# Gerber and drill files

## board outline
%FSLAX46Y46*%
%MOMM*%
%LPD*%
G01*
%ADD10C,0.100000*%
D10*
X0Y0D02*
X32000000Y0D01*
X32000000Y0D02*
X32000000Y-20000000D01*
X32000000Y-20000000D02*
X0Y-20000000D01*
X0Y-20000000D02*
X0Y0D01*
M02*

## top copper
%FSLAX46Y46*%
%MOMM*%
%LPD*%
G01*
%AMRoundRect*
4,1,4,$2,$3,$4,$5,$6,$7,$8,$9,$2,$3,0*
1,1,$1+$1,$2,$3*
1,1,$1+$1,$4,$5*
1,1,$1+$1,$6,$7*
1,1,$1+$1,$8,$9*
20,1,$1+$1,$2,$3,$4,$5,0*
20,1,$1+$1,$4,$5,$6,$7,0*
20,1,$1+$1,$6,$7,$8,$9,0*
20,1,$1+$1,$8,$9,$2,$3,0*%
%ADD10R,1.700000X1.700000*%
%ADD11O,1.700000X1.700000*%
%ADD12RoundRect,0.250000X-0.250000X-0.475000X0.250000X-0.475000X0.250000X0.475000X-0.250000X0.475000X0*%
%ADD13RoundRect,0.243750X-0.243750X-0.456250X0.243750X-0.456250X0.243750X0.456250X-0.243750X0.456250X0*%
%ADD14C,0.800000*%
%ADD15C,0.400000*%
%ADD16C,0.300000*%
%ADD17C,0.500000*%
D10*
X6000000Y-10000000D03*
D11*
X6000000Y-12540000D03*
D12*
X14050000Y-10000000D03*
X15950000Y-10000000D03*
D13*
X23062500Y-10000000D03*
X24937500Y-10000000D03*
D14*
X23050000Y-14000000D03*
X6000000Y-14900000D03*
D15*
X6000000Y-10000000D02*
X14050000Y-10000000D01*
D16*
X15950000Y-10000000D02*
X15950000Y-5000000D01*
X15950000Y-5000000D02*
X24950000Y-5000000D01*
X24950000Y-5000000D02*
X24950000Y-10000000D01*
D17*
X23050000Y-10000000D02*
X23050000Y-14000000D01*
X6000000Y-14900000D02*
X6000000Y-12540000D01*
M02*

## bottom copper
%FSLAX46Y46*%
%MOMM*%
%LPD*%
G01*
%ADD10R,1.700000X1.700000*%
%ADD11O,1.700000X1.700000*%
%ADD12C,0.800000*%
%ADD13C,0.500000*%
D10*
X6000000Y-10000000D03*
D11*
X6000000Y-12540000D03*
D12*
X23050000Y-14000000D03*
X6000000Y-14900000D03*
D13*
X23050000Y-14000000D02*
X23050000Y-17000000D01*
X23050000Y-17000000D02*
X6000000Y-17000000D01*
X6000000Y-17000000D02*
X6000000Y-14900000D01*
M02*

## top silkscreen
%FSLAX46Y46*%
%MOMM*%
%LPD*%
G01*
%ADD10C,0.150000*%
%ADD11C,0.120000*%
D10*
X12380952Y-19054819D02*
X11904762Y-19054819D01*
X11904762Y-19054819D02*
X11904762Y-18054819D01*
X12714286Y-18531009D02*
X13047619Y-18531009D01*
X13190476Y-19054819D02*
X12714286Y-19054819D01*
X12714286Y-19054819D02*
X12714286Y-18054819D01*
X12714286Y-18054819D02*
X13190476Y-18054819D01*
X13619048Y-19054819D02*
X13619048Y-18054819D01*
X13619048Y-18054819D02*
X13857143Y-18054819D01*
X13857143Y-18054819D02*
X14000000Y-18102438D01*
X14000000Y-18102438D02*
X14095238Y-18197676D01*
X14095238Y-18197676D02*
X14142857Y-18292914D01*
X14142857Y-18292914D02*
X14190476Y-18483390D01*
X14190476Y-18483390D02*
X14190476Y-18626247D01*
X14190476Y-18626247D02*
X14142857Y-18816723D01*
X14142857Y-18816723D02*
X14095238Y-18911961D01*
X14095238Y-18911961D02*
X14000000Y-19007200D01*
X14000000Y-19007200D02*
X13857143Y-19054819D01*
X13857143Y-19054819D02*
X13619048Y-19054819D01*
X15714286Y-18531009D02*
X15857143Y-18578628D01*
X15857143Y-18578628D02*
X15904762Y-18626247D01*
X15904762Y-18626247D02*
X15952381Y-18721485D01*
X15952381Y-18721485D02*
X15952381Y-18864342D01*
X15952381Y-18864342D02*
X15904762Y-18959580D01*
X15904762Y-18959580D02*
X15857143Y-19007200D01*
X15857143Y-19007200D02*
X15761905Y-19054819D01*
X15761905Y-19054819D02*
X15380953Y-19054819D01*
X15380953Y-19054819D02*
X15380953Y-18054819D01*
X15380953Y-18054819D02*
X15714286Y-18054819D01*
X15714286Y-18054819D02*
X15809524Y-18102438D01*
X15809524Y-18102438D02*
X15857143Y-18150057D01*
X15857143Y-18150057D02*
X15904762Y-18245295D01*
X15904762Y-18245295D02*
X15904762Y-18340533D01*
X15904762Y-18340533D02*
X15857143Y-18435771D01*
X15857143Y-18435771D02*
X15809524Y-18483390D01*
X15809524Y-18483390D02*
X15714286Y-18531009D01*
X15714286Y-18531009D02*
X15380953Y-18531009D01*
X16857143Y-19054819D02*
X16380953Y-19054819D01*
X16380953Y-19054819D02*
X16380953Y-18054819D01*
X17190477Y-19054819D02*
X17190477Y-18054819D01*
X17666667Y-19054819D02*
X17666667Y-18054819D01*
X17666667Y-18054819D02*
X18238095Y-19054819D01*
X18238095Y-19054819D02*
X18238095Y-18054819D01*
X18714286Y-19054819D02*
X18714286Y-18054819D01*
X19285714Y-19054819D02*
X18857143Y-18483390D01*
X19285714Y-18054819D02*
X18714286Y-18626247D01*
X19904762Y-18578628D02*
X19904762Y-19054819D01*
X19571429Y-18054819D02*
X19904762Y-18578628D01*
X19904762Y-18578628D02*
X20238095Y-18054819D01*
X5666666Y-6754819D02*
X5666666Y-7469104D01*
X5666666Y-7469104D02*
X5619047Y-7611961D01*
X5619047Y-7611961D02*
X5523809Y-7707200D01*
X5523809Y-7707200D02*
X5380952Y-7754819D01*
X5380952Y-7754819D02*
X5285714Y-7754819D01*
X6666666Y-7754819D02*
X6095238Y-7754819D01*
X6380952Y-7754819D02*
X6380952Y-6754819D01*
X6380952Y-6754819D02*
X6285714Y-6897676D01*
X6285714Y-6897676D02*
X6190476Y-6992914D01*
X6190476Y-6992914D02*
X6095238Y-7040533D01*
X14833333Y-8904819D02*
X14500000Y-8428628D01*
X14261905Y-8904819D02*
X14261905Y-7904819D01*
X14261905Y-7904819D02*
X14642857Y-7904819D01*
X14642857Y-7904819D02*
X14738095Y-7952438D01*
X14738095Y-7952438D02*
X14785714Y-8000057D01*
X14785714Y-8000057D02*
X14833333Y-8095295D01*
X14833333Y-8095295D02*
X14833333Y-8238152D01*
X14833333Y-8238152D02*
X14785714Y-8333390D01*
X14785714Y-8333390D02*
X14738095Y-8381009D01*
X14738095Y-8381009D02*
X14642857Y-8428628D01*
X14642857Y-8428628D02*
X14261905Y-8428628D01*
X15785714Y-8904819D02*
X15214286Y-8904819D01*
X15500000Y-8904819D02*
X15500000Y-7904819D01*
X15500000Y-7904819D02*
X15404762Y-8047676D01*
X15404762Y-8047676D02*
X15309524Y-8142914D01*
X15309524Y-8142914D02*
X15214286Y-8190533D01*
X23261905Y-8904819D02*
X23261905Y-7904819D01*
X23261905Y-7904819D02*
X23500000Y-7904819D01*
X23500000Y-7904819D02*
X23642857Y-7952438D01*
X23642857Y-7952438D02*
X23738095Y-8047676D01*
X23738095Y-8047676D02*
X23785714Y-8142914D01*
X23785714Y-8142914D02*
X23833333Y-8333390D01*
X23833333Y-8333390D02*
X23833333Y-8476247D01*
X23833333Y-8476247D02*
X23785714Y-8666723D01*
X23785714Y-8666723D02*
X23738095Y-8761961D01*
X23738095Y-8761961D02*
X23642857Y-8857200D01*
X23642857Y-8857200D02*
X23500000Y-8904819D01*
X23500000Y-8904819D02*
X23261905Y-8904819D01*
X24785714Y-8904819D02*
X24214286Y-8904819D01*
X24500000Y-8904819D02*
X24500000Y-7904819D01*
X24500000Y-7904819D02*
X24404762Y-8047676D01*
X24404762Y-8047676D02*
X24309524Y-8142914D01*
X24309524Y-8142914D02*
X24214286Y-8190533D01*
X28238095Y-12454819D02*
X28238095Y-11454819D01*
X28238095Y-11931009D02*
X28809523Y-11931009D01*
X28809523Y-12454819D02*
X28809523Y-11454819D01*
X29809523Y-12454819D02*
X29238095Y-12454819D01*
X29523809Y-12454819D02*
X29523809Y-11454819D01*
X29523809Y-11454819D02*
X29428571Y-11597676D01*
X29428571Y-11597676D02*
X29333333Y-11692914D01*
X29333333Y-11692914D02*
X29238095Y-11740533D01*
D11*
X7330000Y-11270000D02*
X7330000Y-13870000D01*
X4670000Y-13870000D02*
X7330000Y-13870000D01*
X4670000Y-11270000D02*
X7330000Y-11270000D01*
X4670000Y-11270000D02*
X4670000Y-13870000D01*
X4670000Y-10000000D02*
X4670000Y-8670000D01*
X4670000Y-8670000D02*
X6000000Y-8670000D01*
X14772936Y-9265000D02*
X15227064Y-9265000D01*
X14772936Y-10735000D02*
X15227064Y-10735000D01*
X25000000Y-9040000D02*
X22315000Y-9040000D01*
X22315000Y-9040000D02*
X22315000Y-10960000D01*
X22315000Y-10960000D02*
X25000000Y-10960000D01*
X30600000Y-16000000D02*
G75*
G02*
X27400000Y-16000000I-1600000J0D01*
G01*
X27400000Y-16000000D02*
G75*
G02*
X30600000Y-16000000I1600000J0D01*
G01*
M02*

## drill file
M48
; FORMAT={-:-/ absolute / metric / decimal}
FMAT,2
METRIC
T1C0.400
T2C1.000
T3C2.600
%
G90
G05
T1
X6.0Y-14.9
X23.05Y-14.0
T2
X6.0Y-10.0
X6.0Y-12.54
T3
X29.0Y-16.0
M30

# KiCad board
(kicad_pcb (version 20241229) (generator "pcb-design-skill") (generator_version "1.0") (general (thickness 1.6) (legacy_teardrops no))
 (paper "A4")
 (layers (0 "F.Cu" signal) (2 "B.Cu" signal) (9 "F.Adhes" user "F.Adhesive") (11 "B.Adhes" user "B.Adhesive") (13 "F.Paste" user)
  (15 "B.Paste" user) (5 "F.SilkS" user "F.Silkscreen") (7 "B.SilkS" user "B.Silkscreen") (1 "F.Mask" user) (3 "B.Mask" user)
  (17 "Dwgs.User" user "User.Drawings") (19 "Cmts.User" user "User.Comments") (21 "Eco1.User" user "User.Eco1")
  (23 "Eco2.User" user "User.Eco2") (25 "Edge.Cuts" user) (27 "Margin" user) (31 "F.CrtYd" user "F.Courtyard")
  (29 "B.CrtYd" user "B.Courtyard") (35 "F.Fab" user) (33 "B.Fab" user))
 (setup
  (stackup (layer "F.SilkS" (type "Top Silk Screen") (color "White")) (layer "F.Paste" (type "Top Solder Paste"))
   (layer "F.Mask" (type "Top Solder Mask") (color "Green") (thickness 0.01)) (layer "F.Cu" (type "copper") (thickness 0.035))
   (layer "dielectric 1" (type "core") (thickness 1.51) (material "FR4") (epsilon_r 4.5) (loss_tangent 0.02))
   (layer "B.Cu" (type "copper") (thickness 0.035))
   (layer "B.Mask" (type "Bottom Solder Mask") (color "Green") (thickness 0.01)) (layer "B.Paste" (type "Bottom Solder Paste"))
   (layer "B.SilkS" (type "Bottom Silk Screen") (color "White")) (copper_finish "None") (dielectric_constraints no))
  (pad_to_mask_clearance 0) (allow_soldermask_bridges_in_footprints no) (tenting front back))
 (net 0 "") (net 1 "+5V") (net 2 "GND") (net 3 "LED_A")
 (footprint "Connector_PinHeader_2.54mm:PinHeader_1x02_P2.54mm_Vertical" (layer "F.Cu") (at 6 10 0)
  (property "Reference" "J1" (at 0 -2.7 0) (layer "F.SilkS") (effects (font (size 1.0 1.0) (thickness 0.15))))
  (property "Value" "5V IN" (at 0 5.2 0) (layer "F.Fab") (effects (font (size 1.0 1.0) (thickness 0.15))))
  (fp_line (start 1.33 1.27) (end 1.33 3.87) (stroke (width 0.12) (type solid)) (layer "F.SilkS"))
  (fp_line (start -1.33 3.87) (end 1.33 3.87) (stroke (width 0.12) (type solid)) (layer "F.SilkS"))
  (fp_line (start -1.33 1.27) (end 1.33 1.27) (stroke (width 0.12) (type solid)) (layer "F.SilkS"))
  (fp_line (start -1.33 1.27) (end -1.33 3.87) (stroke (width 0.12) (type solid)) (layer "F.SilkS"))
  (fp_line (start -1.33 0) (end -1.33 -1.33) (stroke (width 0.12) (type solid)) (layer "F.SilkS"))
  (fp_line (start -1.33 -1.33) (end 0 -1.33) (stroke (width 0.12) (type solid)) (layer "F.SilkS"))
  (pad "1" thru_hole rect (at 0 0) (size 1.7 1.7) (drill 1) (layers "*.Cu" "*.Mask") (remove_unused_layers no) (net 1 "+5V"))
  (pad "2" thru_hole oval (at 0 2.54) (size 1.7 1.7) (drill 1) (layers "*.Cu" "*.Mask") (remove_unused_layers no) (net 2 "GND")))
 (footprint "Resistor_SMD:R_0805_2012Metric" (layer "F.Cu") (at 15 10)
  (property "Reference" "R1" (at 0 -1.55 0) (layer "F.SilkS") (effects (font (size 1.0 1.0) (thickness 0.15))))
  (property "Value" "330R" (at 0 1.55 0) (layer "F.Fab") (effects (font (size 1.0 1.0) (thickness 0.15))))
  (fp_line (start -0.227064 -0.735) (end 0.227064 -0.735) (stroke (width 0.12) (type solid)) (layer "F.SilkS"))
  (fp_line (start -0.227064 0.735) (end 0.227064 0.735) (stroke (width 0.12) (type solid)) (layer "F.SilkS"))
  (pad "1" smd roundrect (at -0.95 0) (size 1.0 1.45) (layers "F.Cu" "F.Paste" "F.Mask") (roundrect_rratio 0.25) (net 1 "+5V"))
  (pad "2" smd roundrect (at 0.95 0) (size 1.0 1.45) (layers "F.Cu" "F.Paste" "F.Mask") (roundrect_rratio 0.25) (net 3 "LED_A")))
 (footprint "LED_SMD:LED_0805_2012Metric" (layer "F.Cu") (at 24 10)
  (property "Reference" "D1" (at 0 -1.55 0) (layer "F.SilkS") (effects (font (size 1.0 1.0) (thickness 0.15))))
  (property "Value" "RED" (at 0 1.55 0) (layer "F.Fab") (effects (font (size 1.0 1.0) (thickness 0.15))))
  (fp_line (start 1 -0.96) (end -1.685 -0.96) (stroke (width 0.12) (type solid)) (layer "F.SilkS"))
  (fp_line (start -1.685 -0.96) (end -1.685 0.96) (stroke (width 0.12) (type solid)) (layer "F.SilkS"))
  (fp_line (start -1.685 0.96) (end 1 0.96) (stroke (width 0.12) (type solid)) (layer "F.SilkS"))
  (pad "1" smd roundrect (at -0.9375 0) (size 0.975 1.4) (layers "F.Cu" "F.Paste" "F.Mask") (roundrect_rratio 0.25) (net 2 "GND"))
  (pad "2" smd roundrect (at 0.9375 0) (size 0.975 1.4) (layers "F.Cu" "F.Paste" "F.Mask") (roundrect_rratio 0.25) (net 3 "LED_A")))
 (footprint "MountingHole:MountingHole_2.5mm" (layer "F.Cu") (at 29 16)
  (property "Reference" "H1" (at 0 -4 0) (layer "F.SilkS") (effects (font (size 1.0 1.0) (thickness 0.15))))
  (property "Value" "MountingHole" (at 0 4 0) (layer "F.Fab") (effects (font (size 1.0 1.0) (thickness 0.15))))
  (fp_circle (center 0 0) (end 1.6 0) (stroke (width 0.12) (type solid)) (layer "F.SilkS"))
  (pad "" np_thru_hole circle (at 0 0) (size 2.6 2.6) (drill 2.6) (layers "*.Cu" "*.Mask")))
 (segment (start 6 10) (end 14.05 10) (width 0.4) (layer "F.Cu") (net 1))
 (segment (start 15.95 10) (end 15.95 5) (width 0.3) (layer "F.Cu") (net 3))
 (segment (start 15.95 5) (end 24.95 5) (width 0.3) (layer "F.Cu") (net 3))
 (segment (start 24.95 5) (end 24.95 10) (width 0.3) (layer "F.Cu") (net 3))
 (segment (start 23.05 10) (end 23.05 14) (width 0.5) (layer "F.Cu") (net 2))
 (via (at 23.05 14) (size 0.8) (drill 0.4) (layers "F.Cu" "B.Cu") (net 2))
 (segment (start 23.05 14) (end 23.05 17) (width 0.5) (layer "B.Cu") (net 2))
 (segment (start 23.05 17) (end 6 17) (width 0.5) (layer "B.Cu") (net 2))
 (segment (start 6 17) (end 6 14.9) (width 0.5) (layer "B.Cu") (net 2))
 (via (at 6 14.9) (size 0.8) (drill 0.4) (layers "F.Cu" "B.Cu") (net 2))
 (segment (start 6 14.9) (end 6 12.54) (width 0.5) (layer "F.Cu") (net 2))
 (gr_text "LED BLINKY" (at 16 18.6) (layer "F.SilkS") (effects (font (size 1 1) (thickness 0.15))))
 (gr_line (start 0 0) (end 32 0) (stroke (width 0.1) (type solid)) (layer "Edge.Cuts"))
 (gr_line (start 32 0) (end 32 20) (stroke (width 0.1) (type solid)) (layer "Edge.Cuts"))
 (gr_line (start 32 20) (end 0 20) (stroke (width 0.1) (type solid)) (layer "Edge.Cuts"))
 (gr_line (start 0 20) (end 0 0) (stroke (width 0.1) (type solid)) (layer "Edge.Cuts")))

